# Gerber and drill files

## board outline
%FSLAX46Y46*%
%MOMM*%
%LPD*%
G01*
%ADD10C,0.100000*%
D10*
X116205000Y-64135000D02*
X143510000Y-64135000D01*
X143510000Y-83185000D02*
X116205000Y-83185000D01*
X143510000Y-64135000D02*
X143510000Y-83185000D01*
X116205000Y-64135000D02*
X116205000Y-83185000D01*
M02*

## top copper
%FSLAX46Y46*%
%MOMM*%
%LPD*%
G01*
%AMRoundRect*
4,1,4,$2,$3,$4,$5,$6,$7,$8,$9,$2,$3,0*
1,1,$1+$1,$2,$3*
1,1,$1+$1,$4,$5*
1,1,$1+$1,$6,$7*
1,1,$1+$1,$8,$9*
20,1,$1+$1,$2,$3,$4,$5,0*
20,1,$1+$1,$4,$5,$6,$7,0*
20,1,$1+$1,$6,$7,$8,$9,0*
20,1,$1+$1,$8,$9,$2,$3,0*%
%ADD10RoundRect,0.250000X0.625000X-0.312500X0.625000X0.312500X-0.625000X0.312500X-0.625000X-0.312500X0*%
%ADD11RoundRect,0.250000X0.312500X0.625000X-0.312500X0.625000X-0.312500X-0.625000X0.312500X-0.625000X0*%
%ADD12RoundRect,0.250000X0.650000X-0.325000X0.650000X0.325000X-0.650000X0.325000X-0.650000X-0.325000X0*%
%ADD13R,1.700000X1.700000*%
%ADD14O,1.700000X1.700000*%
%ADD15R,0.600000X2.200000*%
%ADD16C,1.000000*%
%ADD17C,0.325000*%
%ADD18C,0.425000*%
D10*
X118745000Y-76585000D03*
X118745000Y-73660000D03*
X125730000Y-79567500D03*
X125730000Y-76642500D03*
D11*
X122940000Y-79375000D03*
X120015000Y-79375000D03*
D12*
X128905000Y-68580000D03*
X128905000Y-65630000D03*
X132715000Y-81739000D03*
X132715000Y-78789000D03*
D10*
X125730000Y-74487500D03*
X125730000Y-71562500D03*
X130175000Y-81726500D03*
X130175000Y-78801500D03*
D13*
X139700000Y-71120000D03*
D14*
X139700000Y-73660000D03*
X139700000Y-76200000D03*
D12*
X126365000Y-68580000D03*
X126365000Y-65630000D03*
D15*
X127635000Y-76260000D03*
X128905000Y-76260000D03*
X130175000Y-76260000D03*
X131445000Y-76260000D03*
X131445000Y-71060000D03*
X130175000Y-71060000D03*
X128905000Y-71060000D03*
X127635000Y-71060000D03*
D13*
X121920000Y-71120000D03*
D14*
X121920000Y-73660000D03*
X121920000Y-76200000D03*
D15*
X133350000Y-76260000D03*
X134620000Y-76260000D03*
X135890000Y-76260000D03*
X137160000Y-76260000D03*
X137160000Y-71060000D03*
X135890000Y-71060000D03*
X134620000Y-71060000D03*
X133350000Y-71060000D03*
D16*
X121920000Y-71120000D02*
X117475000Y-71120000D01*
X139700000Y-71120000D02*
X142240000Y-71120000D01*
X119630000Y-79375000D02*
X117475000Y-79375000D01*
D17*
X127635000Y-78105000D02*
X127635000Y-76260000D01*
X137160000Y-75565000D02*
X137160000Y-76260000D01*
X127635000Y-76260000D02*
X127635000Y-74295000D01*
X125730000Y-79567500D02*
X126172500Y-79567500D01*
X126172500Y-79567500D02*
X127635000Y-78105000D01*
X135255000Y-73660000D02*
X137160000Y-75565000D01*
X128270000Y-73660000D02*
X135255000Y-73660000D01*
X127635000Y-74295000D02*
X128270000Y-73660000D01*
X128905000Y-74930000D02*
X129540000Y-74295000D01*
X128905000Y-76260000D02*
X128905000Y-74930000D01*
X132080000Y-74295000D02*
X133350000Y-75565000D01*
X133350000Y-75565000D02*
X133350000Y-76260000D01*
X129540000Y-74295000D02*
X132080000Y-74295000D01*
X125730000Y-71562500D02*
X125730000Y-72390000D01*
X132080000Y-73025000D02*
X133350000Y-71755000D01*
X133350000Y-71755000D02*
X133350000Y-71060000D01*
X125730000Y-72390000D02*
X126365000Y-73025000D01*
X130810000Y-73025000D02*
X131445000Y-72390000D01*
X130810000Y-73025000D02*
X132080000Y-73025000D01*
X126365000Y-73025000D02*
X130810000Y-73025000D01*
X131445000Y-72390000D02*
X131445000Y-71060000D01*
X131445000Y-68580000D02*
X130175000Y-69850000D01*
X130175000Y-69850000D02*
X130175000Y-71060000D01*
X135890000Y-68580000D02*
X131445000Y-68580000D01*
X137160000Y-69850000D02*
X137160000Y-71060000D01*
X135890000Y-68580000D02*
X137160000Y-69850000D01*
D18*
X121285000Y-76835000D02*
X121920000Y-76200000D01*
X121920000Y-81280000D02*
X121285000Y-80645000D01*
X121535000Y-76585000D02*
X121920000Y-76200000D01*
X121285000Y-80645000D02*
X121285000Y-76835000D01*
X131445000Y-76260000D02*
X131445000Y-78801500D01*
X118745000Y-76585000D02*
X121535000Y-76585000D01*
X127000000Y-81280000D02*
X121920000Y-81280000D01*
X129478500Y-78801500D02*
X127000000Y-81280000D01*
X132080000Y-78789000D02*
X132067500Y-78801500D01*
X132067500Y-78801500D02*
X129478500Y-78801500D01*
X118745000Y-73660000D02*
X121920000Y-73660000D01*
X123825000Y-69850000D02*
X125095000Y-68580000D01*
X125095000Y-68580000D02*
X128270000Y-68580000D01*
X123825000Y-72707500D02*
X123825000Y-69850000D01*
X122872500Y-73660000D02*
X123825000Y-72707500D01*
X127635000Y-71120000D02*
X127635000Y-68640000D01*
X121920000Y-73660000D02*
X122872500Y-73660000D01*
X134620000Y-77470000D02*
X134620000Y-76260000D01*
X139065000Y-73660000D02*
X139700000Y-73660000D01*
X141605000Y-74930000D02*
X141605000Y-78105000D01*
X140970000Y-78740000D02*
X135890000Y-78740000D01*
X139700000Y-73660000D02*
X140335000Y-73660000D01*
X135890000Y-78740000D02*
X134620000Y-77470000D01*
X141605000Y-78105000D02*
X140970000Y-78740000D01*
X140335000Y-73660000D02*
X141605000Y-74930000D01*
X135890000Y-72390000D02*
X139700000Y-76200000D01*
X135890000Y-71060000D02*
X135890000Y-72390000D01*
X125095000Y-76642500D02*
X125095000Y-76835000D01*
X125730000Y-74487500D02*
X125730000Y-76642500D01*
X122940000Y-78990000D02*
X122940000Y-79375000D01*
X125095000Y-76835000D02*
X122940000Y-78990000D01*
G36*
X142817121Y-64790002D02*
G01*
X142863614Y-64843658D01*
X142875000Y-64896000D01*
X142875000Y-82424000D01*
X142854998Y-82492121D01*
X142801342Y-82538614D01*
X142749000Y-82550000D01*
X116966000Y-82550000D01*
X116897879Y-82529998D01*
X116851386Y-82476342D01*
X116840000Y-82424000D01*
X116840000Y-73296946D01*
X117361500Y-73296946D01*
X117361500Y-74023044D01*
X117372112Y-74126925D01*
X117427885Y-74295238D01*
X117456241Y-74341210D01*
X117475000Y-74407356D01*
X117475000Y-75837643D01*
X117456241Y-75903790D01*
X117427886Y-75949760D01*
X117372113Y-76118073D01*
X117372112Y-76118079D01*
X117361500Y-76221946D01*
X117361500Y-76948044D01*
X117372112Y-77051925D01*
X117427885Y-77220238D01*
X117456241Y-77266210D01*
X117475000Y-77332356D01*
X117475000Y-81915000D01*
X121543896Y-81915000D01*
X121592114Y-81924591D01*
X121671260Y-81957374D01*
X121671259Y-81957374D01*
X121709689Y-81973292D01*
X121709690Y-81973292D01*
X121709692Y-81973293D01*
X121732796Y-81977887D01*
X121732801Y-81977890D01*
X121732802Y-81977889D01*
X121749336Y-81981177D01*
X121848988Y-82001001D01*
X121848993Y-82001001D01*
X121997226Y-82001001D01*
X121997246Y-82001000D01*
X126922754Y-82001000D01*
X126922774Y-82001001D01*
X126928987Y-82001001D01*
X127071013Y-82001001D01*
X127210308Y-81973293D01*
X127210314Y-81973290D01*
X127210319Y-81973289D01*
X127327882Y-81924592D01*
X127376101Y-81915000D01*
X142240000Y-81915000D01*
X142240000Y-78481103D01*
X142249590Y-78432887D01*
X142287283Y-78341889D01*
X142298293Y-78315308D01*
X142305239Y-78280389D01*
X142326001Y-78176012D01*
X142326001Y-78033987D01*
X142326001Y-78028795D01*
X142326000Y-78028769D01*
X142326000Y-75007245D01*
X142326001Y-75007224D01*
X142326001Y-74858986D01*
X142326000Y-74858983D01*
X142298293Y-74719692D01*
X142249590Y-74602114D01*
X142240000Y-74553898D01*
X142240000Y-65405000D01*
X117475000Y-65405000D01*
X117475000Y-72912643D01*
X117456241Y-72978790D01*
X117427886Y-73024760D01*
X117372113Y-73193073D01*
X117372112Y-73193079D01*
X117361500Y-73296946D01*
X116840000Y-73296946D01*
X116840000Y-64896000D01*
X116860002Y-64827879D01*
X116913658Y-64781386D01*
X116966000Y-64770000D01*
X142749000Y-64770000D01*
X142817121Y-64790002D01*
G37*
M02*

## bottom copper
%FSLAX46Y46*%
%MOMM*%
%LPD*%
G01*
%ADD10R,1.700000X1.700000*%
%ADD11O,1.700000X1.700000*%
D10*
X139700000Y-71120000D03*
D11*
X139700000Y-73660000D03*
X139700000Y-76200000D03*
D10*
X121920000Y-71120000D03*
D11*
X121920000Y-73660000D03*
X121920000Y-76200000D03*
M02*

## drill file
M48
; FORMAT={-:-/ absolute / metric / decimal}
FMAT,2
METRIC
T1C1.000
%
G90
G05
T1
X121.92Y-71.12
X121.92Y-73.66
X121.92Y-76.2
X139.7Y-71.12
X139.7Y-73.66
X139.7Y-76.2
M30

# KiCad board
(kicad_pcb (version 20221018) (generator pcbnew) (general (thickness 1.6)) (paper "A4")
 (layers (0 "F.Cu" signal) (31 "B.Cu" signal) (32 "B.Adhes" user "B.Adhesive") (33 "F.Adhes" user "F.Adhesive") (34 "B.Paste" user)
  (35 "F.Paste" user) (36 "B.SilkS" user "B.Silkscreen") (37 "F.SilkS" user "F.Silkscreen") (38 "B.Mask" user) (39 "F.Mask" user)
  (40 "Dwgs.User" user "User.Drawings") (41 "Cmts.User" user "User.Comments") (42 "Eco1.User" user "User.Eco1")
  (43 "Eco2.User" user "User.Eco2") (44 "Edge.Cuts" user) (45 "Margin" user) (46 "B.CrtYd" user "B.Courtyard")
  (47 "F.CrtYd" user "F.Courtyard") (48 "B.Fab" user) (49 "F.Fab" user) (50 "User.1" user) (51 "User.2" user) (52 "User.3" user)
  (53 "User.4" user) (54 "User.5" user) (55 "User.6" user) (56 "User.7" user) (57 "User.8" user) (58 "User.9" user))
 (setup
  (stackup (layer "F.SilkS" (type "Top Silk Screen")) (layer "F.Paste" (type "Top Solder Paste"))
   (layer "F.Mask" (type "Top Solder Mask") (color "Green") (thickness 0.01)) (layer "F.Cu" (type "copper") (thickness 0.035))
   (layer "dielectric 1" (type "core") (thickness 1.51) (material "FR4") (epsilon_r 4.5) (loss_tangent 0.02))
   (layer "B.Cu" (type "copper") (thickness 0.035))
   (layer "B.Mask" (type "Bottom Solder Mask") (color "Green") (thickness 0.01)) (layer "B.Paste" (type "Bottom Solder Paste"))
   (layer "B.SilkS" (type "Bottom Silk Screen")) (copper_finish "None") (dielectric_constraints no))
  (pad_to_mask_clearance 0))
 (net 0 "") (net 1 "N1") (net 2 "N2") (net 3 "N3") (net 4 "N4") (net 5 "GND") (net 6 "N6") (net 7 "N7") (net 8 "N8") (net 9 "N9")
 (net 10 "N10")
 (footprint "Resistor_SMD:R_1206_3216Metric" (layer "F.Cu") (at 118.745 75.1225 90)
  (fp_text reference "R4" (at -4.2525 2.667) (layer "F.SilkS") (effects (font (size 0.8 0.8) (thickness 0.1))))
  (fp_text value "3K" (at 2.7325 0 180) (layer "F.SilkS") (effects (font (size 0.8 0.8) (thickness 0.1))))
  (pad "1" smd roundrect (at -1.4625 0 90) (size 1.125 1.75) (layers "F.Cu" "F.Paste" "F.Mask") (roundrect_rratio 0.2222222222) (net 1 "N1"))
  (pad "2" smd roundrect (at 1.4625 0 90) (size 1.125 1.75) (layers "F.Cu" "F.Paste" "F.Mask") (roundrect_rratio 0.2222222222) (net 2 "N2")))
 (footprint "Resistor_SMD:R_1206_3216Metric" (layer "F.Cu") (at 125.73 78.105 90)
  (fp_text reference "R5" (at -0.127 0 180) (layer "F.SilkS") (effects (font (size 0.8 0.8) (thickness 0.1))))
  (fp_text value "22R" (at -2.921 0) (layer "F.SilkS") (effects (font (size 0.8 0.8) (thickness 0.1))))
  (pad "1" smd roundrect (at -1.4625 0 90) (size 1.125 1.75) (layers "F.Cu" "F.Paste" "F.Mask") (roundrect_rratio 0.2222222222) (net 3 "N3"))
  (pad "2" smd roundrect (at 1.4625 0 90) (size 1.125 1.75) (layers "F.Cu" "F.Paste" "F.Mask") (roundrect_rratio 0.2222222222) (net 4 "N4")))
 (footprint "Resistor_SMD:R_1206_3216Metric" (layer "F.Cu") (at 121.4775 79.375 180)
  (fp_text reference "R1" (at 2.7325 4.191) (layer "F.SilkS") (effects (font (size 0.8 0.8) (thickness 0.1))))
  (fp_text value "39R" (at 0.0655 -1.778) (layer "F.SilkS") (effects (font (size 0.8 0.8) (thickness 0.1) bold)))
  (pad "1" smd roundrect (at -1.4625 0 180) (size 1.125 1.75) (layers "F.Cu" "F.Paste" "F.Mask") (roundrect_rratio 0.2222222222)
   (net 4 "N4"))
  (pad "2" smd roundrect (at 1.4625 0 180) (size 1.125 1.75) (layers "F.Cu" "F.Paste" "F.Mask") (roundrect_rratio 0.2222222222)
   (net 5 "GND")))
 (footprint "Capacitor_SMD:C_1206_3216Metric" (layer "F.Cu") (at 128.905 67.105 90)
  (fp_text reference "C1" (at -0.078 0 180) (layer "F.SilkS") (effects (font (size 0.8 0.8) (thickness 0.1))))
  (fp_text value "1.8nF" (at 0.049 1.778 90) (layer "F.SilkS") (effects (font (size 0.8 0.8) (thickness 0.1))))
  (pad "1" smd roundrect (at -1.475 0 90) (size 1.15 1.8) (layers "F.Cu" "F.Paste" "F.Mask") (roundrect_rratio 0.2173913043) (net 2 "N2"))
  (pad "2" smd roundrect (at 1.475 0 90) (size 1.15 1.8) (layers "F.Cu" "F.Paste" "F.Mask") (roundrect_rratio 0.2173913043) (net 5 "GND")))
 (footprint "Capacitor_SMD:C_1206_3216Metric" (layer "F.Cu") (at 132.715 80.264 90)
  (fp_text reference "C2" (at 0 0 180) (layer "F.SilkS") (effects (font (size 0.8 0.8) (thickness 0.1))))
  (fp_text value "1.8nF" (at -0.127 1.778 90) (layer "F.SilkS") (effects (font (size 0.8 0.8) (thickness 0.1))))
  (pad "1" smd roundrect (at -1.475 0 90) (size 1.15 1.8) (layers "F.Cu" "F.Paste" "F.Mask") (roundrect_rratio 0.2173913043) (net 5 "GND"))
  (pad "2" smd roundrect (at 1.475 0 90) (size 1.15 1.8) (layers "F.Cu" "F.Paste" "F.Mask") (roundrect_rratio 0.2173913043) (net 1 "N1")))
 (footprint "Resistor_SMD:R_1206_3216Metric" (layer "F.Cu") (at 125.73 73.025 90)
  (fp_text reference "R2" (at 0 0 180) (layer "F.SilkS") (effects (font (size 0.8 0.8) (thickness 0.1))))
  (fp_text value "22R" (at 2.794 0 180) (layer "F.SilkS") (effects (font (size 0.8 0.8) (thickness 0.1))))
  (pad "1" smd roundrect (at -1.4625 0 90) (size 1.125 1.75) (layers "F.Cu" "F.Paste" "F.Mask") (roundrect_rratio 0.2222222222) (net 4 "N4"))
  (pad "2" smd roundrect (at 1.4625 0 90) (size 1.125 1.75) (layers "F.Cu" "F.Paste" "F.Mask") (roundrect_rratio 0.2222222222) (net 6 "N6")))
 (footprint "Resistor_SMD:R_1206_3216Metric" (layer "F.Cu") (at 130.175 80.264 90)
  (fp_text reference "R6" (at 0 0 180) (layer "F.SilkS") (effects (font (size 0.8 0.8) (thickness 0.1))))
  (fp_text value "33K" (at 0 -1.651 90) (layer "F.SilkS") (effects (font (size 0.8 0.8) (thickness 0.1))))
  (pad "1" smd roundrect (at -1.4625 0 90) (size 1.125 1.75) (layers "F.Cu" "F.Paste" "F.Mask") (roundrect_rratio 0.2222222222)
   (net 5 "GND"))
  (pad "2" smd roundrect (at 1.4625 0 90) (size 1.125 1.75) (layers "F.Cu" "F.Paste" "F.Mask") (roundrect_rratio 0.2222222222) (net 1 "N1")))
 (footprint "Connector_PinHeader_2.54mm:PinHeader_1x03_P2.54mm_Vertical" (layer "F.Cu") (at 139.7 71.12)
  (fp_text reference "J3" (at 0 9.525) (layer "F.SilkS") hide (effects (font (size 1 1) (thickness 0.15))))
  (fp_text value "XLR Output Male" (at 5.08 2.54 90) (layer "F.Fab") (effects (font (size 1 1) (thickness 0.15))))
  (pad "1" thru_hole rect (at 0 0) (size 1.7 1.7) (drill 1) (layers "*.Cu" "*.Mask") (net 5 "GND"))
  (pad "2" thru_hole oval (at 0 2.54) (size 1.7 1.7) (drill 1) (layers "*.Cu" "*.Mask") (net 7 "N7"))
  (pad "3" thru_hole oval (at 0 5.08) (size 1.7 1.7) (drill 1) (layers "*.Cu" "*.Mask") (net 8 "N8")))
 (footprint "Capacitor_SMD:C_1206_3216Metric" (layer "F.Cu") (at 126.365 67.105 90)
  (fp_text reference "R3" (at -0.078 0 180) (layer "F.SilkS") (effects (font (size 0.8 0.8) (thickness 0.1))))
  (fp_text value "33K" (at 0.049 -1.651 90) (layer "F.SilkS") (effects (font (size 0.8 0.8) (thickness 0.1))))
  (pad "1" smd roundrect (at -1.475 0 90) (size 1.15 1.8) (layers "F.Cu" "F.Paste" "F.Mask") (roundrect_rratio 0.2173913043) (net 2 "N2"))
  (pad "2" smd roundrect (at 1.475 0 90) (size 1.15 1.8) (layers "F.Cu" "F.Paste" "F.Mask") (roundrect_rratio 0.2173913043) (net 5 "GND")))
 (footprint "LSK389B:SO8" (layer "F.Cu") (at 129.54 73.66)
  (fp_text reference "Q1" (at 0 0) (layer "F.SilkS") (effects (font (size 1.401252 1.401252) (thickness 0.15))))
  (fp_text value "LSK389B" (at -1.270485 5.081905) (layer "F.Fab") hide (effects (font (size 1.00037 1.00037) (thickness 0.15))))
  (pad "1" smd rect (at -1.905 2.6) (size 0.6 2.2) (layers "F.Cu" "F.Paste" "F.Mask") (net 3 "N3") (solder_mask_margin 0.102))
  (pad "2" smd rect (at -0.635 2.6) (size 0.6 2.2) (layers "F.Cu" "F.Paste" "F.Mask") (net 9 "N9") (solder_mask_margin 0.102))
  (pad "3" smd rect (at 0.635 2.6) (size 0.6 2.2) (layers "F.Cu" "F.Paste" "F.Mask") (solder_mask_margin 0.102))
  (pad "4" smd rect (at 1.905 2.6) (size 0.6 2.2) (layers "F.Cu" "F.Paste" "F.Mask") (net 1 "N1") (solder_mask_margin 0.102))
  (pad "5" smd rect (at 1.905 -2.6) (size 0.6 2.2) (layers "F.Cu" "F.Paste" "F.Mask") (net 6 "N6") (solder_mask_margin 0.102))
  (pad "6" smd rect (at 0.635 -2.6) (size 0.6 2.2) (layers "F.Cu" "F.Paste" "F.Mask") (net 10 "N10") (solder_mask_margin 0.102))
  (pad "7" smd rect (at -0.635 -2.6) (size 0.6 2.2) (layers "F.Cu" "F.Paste" "F.Mask") (solder_mask_margin 0.102))
  (pad "8" smd rect (at -1.905 -2.6) (size 0.6 2.2) (layers "F.Cu" "F.Paste" "F.Mask") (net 2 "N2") (solder_mask_margin 0.102)))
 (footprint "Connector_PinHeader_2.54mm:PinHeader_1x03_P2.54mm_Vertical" (layer "F.Cu") (at 121.92 71.12)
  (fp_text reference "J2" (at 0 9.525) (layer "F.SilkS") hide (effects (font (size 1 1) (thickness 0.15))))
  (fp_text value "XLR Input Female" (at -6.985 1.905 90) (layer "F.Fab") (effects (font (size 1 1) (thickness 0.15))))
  (pad "1" thru_hole rect (at 0 0) (size 1.7 1.7) (drill 1) (layers "*.Cu" "*.Mask") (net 5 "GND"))
  (pad "2" thru_hole oval (at 0 2.54) (size 1.7 1.7) (drill 1) (layers "*.Cu" "*.Mask") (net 2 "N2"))
  (pad "3" thru_hole oval (at 0 5.08) (size 1.7 1.7) (drill 1) (layers "*.Cu" "*.Mask") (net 1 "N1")))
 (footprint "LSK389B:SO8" (layer "F.Cu") (at 135.255 73.66)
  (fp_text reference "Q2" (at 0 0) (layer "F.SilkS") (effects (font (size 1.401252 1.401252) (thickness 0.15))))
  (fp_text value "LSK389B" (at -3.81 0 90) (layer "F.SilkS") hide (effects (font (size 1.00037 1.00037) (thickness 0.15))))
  (pad "1" smd rect (at -1.905 2.6) (size 0.6 2.2) (layers "F.Cu" "F.Paste" "F.Mask") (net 9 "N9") (solder_mask_margin 0.102))
  (pad "2" smd rect (at -0.635 2.6) (size 0.6 2.2) (layers "F.Cu" "F.Paste" "F.Mask") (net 7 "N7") (solder_mask_margin 0.102))
  (pad "3" smd rect (at 0.635 2.6) (size 0.6 2.2) (layers "F.Cu" "F.Paste" "F.Mask") (solder_mask_margin 0.102))
  (pad "4" smd rect (at 1.905 2.6) (size 0.6 2.2) (layers "F.Cu" "F.Paste" "F.Mask") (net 3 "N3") (solder_mask_margin 0.102))
  (pad "5" smd rect (at 1.905 -2.6) (size 0.6 2.2) (layers "F.Cu" "F.Paste" "F.Mask") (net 10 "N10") (solder_mask_margin 0.102))
  (pad "6" smd rect (at 0.635 -2.6) (size 0.6 2.2) (layers "F.Cu" "F.Paste" "F.Mask") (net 8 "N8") (solder_mask_margin 0.102))
  (pad "7" smd rect (at -0.635 -2.6) (size 0.6 2.2) (layers "F.Cu" "F.Paste" "F.Mask") (solder_mask_margin 0.102))
  (pad "8" smd rect (at -1.905 -2.6) (size 0.6 2.2) (layers "F.Cu" "F.Paste" "F.Mask") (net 6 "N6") (solder_mask_margin 0.102)))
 (gr_line (start 116.205 64.135) (end 143.51 64.135) (stroke (width 0.1) (type solid)) (layer "Edge.Cuts"))
 (gr_line (start 143.51 83.185) (end 116.205 83.185) (stroke (width 0.1) (type solid)) (layer "Edge.Cuts"))
 (gr_line (start 143.51 64.135) (end 143.51 83.185) (stroke (width 0.1) (type default)) (layer "Edge.Cuts"))
 (gr_line (start 116.205 64.135) (end 116.205 83.185) (stroke (width 0.1) (type default)) (layer "Edge.Cuts"))
 (segment (start 121.92 71.12) (end 117.475 71.12) (width 1) (layer "F.Cu") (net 5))
 (segment (start 139.7 71.12) (end 142.24 71.12) (width 1) (layer "F.Cu") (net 5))
 (segment (start 119.63 79.375) (end 117.475 79.375) (width 1) (layer "F.Cu") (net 5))
 (segment (start 127.635 78.105) (end 127.635 76.26) (width 0.325) (layer "F.Cu") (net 3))
 (segment (start 137.16 75.565) (end 137.16 76.26) (width 0.325) (layer "F.Cu") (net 3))
 (segment (start 127.635 76.26) (end 127.635 74.295) (width 0.325) (layer "F.Cu") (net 3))
 (segment (start 125.73 79.5675) (end 126.1725 79.5675) (width 0.325) (layer "F.Cu") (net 3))
 (segment (start 126.1725 79.5675) (end 127.635 78.105) (width 0.325) (layer "F.Cu") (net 3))
 (segment (start 135.255 73.66) (end 137.16 75.565) (width 0.325) (layer "F.Cu") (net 3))
 (segment (start 128.27 73.66) (end 135.255 73.66) (width 0.325) (layer "F.Cu") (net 3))
 (segment (start 127.635 74.295) (end 128.27 73.66) (width 0.325) (layer "F.Cu") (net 3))
 (segment (start 128.905 74.93) (end 129.54 74.295) (width 0.325) (layer "F.Cu") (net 9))
 (segment (start 128.905 76.26) (end 128.905 74.93) (width 0.325) (layer "F.Cu") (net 9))
 (segment (start 132.08 74.295) (end 133.35 75.565) (width 0.325) (layer "F.Cu") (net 9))
 (segment (start 133.35 75.565) (end 133.35 76.26) (width 0.325) (layer "F.Cu") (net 9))
 (segment (start 129.54 74.295) (end 132.08 74.295) (width 0.325) (layer "F.Cu") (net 9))
 (segment (start 125.73 71.5625) (end 125.73 72.39) (width 0.325) (layer "F.Cu") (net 6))
 (segment (start 132.08 73.025) (end 133.35 71.755) (width 0.325) (layer "F.Cu") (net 6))
 (segment (start 133.35 71.755) (end 133.35 71.06) (width 0.325) (layer "F.Cu") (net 6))
 (segment (start 125.73 72.39) (end 126.365 73.025) (width 0.325) (layer "F.Cu") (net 6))
 (segment (start 130.81 73.025) (end 131.445 72.39) (width 0.325) (layer "F.Cu") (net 6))
 (segment (start 130.81 73.025) (end 132.08 73.025) (width 0.325) (layer "F.Cu") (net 6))
 (segment (start 126.365 73.025) (end 130.81 73.025) (width 0.325) (layer "F.Cu") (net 6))
 (segment (start 131.445 72.39) (end 131.445 71.06) (width 0.325) (layer "F.Cu") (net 6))
 (segment (start 131.445 68.58) (end 130.175 69.85) (width 0.325) (layer "F.Cu") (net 10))
 (segment (start 130.175 69.85) (end 130.175 71.06) (width 0.325) (layer "F.Cu") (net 10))
 (segment (start 135.89 68.58) (end 131.445 68.58) (width 0.325) (layer "F.Cu") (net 10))
 (segment (start 137.16 69.85) (end 137.16 71.06) (width 0.325) (layer "F.Cu") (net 10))
 (segment (start 135.89 68.58) (end 137.16 69.85) (width 0.325) (layer "F.Cu") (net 10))
 (segment (start 121.285 76.835) (end 121.92 76.2) (width 0.425) (layer "F.Cu") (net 1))
 (segment (start 121.92 81.28) (end 121.285 80.645) (width 0.425) (layer "F.Cu") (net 1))
 (segment (start 121.535 76.585) (end 121.92 76.2) (width 0.425) (layer "F.Cu") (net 1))
 (segment (start 121.285 80.645) (end 121.285 76.835) (width 0.425) (layer "F.Cu") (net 1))
 (segment (start 131.445 76.26) (end 131.445 78.8015) (width 0.425) (layer "F.Cu") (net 1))
 (segment (start 118.745 76.585) (end 121.535 76.585) (width 0.425) (layer "F.Cu") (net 1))
 (segment (start 127 81.28) (end 121.92 81.28) (width 0.425) (layer "F.Cu") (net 1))
 (segment (start 129.4785 78.8015) (end 127 81.28) (width 0.425) (layer "F.Cu") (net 1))
 (segment (start 132.08 78.789) (end 132.0675 78.8015) (width 0.425) (layer "F.Cu") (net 1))
 (segment (start 132.0675 78.8015) (end 129.4785 78.8015) (width 0.425) (layer "F.Cu") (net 1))
 (segment (start 118.745 73.66) (end 121.92 73.66) (width 0.425) (layer "F.Cu") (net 2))
 (segment (start 123.825 69.85) (end 125.095 68.58) (width 0.425) (layer "F.Cu") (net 2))
 (segment (start 125.095 68.58) (end 128.27 68.58) (width 0.425) (layer "F.Cu") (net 2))
 (segment (start 123.825 72.7075) (end 123.825 69.85) (width 0.425) (layer "F.Cu") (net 2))
 (segment (start 122.8725 73.66) (end 123.825 72.7075) (width 0.425) (layer "F.Cu") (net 2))
 (segment (start 127.635 71.12) (end 127.635 68.64) (width 0.425) (layer "F.Cu") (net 2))
 (segment (start 121.92 73.66) (end 122.8725 73.66) (width 0.425) (layer "F.Cu") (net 2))
 (segment (start 134.62 77.47) (end 134.62 76.26) (width 0.425) (layer "F.Cu") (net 7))
 (segment (start 139.065 73.66) (end 139.7 73.66) (width 0.425) (layer "F.Cu") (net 7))
 (segment (start 141.605 74.93) (end 141.605 78.105) (width 0.425) (layer "F.Cu") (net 7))
 (segment (start 140.97 78.74) (end 135.89 78.74) (width 0.425) (layer "F.Cu") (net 7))
 (segment (start 139.7 73.66) (end 140.335 73.66) (width 0.425) (layer "F.Cu") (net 7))
 (segment (start 135.89 78.74) (end 134.62 77.47) (width 0.425) (layer "F.Cu") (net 7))
 (segment (start 141.605 78.105) (end 140.97 78.74) (width 0.425) (layer "F.Cu") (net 7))
 (segment (start 140.335 73.66) (end 141.605 74.93) (width 0.425) (layer "F.Cu") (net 7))
 (segment (start 135.89 72.39) (end 139.7 76.2) (width 0.425) (layer "F.Cu") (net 8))
 (segment (start 135.89 71.06) (end 135.89 72.39) (width 0.425) (layer "F.Cu") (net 8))
 (segment (start 125.095 76.6425) (end 125.095 76.835) (width 0.425) (layer "F.Cu") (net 4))
 (segment (start 125.73 74.4875) (end 125.73 76.6425) (width 0.425) (layer "F.Cu") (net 4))
 (segment (start 122.94 78.99) (end 122.94 79.375) (width 0.425) (layer "F.Cu") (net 4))
 (segment (start 125.095 76.835) (end 122.94 78.99) (width 0.425) (layer "F.Cu") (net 4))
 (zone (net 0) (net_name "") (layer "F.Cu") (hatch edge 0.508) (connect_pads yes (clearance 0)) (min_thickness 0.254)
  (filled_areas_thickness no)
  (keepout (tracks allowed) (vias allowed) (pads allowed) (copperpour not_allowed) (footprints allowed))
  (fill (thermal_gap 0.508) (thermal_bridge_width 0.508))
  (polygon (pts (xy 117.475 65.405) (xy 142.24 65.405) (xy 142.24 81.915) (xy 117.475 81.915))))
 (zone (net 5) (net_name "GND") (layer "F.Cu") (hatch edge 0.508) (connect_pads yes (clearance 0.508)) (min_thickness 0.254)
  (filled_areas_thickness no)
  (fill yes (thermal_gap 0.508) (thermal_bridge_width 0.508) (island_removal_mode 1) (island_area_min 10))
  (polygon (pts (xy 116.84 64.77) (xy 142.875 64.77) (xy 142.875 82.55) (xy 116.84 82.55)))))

